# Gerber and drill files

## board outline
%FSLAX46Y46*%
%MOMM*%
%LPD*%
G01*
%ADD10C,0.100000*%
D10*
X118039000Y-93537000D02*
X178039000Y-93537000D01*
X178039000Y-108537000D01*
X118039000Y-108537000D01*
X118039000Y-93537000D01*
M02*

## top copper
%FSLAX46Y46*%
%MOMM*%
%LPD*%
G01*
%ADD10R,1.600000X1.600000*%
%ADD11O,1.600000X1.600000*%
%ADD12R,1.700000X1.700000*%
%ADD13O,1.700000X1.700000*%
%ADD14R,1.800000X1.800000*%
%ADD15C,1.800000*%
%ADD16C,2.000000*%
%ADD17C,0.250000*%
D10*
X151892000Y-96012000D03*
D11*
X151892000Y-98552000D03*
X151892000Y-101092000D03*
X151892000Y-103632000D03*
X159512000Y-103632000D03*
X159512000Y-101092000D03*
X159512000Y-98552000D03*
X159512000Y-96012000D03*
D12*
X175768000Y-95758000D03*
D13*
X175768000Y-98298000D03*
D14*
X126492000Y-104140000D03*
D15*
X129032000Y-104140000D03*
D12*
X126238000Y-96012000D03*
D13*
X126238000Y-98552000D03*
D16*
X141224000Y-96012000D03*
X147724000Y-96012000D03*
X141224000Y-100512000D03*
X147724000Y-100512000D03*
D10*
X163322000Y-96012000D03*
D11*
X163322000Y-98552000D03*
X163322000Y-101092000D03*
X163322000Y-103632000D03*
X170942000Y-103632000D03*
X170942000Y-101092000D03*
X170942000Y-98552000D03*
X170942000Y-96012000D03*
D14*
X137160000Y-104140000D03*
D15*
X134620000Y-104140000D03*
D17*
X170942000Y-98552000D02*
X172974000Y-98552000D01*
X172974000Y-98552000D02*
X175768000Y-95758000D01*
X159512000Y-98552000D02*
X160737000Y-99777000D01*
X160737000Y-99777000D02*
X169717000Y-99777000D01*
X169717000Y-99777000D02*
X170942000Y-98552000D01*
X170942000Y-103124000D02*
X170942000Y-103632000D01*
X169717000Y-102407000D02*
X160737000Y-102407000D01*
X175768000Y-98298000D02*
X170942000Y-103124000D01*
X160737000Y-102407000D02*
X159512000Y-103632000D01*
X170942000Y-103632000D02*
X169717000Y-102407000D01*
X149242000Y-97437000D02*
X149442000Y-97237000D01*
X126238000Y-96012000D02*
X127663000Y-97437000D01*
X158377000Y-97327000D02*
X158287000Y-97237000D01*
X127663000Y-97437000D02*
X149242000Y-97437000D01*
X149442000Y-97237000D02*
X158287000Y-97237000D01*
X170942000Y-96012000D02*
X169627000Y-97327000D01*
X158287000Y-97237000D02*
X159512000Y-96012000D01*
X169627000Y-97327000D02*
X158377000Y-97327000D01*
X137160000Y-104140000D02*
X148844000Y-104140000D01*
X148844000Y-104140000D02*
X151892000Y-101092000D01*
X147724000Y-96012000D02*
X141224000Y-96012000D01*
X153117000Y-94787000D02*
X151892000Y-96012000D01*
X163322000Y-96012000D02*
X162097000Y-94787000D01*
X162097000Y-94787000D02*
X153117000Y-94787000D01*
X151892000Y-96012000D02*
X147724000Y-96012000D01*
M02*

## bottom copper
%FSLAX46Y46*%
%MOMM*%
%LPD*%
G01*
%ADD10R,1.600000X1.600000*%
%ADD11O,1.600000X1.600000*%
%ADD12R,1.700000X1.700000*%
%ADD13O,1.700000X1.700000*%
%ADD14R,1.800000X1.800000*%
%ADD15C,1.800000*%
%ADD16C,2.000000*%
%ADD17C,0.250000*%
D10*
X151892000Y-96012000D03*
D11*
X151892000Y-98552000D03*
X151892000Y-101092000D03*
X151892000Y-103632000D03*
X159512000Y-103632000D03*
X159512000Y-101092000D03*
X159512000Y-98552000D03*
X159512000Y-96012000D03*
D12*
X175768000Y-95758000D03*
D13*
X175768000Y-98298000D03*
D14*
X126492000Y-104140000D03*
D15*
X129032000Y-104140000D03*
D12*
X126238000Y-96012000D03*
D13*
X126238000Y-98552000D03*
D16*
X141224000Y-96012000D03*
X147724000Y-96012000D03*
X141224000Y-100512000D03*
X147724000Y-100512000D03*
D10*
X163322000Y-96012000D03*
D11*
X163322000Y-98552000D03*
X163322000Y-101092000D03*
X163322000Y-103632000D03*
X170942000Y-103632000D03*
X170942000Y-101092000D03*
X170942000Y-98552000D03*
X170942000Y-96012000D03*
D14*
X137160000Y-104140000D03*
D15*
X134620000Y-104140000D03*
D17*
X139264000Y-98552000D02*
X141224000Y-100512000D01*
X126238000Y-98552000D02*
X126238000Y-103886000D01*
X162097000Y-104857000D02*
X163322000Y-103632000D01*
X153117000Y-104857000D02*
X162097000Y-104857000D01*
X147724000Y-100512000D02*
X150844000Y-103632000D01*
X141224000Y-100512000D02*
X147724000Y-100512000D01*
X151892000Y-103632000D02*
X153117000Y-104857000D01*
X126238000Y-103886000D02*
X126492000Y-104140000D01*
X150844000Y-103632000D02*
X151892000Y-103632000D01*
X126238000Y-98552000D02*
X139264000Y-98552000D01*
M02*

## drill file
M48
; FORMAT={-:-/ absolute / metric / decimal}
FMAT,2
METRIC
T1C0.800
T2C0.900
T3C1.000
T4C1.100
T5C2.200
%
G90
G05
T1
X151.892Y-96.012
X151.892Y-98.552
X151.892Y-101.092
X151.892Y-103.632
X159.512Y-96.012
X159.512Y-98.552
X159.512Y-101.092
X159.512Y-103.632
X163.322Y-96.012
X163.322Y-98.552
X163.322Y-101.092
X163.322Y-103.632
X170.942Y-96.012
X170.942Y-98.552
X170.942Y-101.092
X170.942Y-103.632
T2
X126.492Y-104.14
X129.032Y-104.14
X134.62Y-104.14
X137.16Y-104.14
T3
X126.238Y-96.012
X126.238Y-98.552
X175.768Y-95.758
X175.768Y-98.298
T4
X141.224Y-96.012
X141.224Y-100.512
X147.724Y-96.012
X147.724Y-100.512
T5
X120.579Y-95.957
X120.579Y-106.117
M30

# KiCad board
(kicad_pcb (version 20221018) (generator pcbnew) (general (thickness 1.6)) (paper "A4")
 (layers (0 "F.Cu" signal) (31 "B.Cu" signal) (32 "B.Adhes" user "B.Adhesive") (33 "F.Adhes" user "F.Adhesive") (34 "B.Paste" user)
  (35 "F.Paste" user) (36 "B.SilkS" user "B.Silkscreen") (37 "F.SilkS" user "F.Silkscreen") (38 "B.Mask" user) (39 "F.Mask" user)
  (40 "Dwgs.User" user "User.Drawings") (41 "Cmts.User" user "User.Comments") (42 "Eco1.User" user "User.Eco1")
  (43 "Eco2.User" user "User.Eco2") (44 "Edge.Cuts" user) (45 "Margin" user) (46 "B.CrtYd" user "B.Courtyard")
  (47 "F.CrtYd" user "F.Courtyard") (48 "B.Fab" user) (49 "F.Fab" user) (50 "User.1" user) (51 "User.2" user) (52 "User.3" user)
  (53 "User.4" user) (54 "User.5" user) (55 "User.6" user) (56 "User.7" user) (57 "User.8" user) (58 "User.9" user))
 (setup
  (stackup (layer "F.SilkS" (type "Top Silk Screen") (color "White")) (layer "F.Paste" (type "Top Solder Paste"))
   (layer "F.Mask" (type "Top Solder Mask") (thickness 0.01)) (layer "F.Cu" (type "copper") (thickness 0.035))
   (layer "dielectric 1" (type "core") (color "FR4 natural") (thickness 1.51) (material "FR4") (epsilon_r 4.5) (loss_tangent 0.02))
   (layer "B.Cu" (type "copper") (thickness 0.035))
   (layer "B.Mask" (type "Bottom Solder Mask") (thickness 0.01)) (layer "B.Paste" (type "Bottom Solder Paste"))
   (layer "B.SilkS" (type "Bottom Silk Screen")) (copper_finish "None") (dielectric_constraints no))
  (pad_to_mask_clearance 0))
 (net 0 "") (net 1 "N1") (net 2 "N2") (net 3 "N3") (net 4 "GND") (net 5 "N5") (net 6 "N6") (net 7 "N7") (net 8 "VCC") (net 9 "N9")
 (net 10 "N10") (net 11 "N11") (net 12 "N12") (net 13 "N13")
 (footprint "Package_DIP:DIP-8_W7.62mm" (layer "F.Cu") (at 151.892 96.012)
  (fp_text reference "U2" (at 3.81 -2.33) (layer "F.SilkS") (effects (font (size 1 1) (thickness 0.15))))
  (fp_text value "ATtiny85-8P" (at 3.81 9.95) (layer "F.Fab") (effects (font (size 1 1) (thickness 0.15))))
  (pad "1" thru_hole rect (at 0 0) (size 1.6 1.6) (drill 0.8) (layers "*.Cu" "*.Mask") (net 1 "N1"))
  (pad "2" thru_hole oval (at 0 2.54) (size 1.6 1.6) (drill 0.8) (layers "*.Cu" "*.Mask") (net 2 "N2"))
  (pad "3" thru_hole oval (at 0 5.08) (size 1.6 1.6) (drill 0.8) (layers "*.Cu" "*.Mask") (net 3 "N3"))
  (pad "4" thru_hole oval (at 0 7.62) (size 1.6 1.6) (drill 0.8) (layers "*.Cu" "*.Mask") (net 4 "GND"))
  (pad "5" thru_hole oval (at 7.62 7.62) (size 1.6 1.6) (drill 0.8) (layers "*.Cu" "*.Mask") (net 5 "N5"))
  (pad "6" thru_hole oval (at 7.62 5.08) (size 1.6 1.6) (drill 0.8) (layers "*.Cu" "*.Mask") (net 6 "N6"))
  (pad "7" thru_hole oval (at 7.62 2.54) (size 1.6 1.6) (drill 0.8) (layers "*.Cu" "*.Mask") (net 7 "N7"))
  (pad "8" thru_hole oval (at 7.62 0) (size 1.6 1.6) (drill 0.8) (layers "*.Cu" "*.Mask") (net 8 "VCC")))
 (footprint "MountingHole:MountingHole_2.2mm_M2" (layer "F.Cu") (at 120.579 95.957 -90)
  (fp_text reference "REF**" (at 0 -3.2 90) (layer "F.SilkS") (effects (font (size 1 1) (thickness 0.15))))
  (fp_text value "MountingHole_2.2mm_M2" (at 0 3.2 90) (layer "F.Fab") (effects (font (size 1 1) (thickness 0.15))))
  (pad "" np_thru_hole circle (at 0 0 270) (size 2.2 2.2) (drill 2.2) (layers "*.Cu" "*.Mask")))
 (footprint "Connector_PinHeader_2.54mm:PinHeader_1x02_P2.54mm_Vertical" (layer "F.Cu") (at 175.768 95.758)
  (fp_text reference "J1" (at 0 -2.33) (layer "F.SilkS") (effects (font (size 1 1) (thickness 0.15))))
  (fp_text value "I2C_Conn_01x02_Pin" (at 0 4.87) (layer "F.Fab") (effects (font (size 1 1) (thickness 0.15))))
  (pad "1" thru_hole rect (at 0 0) (size 1.7 1.7) (drill 1) (layers "*.Cu" "*.Mask") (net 7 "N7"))
  (pad "2" thru_hole oval (at 0 2.54) (size 1.7 1.7) (drill 1) (layers "*.Cu" "*.Mask") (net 5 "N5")))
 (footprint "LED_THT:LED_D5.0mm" (layer "F.Cu") (at 126.492 104.14)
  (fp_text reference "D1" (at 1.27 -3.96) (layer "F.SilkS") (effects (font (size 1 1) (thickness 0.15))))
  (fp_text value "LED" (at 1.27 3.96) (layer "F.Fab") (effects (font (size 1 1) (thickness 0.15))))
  (pad "1" thru_hole rect (at 0 0) (size 1.8 1.8) (drill 0.9) (layers "*.Cu" "*.Mask") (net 4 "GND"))
  (pad "2" thru_hole circle (at 2.54 0) (size 1.8 1.8) (drill 0.9) (layers "*.Cu" "*.Mask") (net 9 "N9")))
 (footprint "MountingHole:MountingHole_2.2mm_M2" (layer "F.Cu") (at 120.579 106.117 -90)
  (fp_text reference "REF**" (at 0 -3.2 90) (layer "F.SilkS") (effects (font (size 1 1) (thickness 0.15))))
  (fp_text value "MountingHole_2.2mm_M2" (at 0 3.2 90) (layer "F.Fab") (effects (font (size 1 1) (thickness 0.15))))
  (pad "" np_thru_hole circle (at 0 0 270) (size 2.2 2.2) (drill 2.2) (layers "F&B.Cu" "*.Mask")))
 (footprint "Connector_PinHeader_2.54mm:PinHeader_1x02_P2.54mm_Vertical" (layer "F.Cu") (at 126.238 96.012)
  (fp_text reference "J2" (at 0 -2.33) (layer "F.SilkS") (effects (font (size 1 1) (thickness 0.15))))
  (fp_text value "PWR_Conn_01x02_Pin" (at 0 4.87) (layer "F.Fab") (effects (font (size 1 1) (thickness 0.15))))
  (pad "1" thru_hole rect (at 0 0) (size 1.7 1.7) (drill 1) (layers "*.Cu" "*.Mask") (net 8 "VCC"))
  (pad "2" thru_hole oval (at 0 2.54) (size 1.7 1.7) (drill 1) (layers "*.Cu" "*.Mask") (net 4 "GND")))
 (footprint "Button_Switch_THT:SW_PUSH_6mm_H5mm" (layer "F.Cu") (at 141.224 96.012)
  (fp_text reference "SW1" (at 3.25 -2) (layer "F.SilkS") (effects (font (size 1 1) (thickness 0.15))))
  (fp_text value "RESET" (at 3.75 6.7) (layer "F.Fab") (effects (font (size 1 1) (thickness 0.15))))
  (pad "1" thru_hole circle (at 0 0 90) (size 2 2) (drill 1.1) (layers "*.Cu" "*.Mask") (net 1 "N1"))
  (pad "1" thru_hole circle (at 6.5 0 90) (size 2 2) (drill 1.1) (layers "*.Cu" "*.Mask") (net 1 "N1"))
  (pad "2" thru_hole circle (at 0 4.5 90) (size 2 2) (drill 1.1) (layers "*.Cu" "*.Mask") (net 4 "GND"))
  (pad "2" thru_hole circle (at 6.5 4.5 90) (size 2 2) (drill 1.1) (layers "*.Cu" "*.Mask") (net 4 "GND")))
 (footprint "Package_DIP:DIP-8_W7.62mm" (layer "F.Cu") (at 163.322 96.012)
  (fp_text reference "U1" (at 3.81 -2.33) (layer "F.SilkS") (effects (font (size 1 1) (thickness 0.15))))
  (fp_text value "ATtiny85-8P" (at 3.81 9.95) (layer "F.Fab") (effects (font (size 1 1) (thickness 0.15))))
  (pad "1" thru_hole rect (at 0 0) (size 1.6 1.6) (drill 0.8) (layers "*.Cu" "*.Mask") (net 1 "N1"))
  (pad "2" thru_hole oval (at 0 2.54) (size 1.6 1.6) (drill 0.8) (layers "*.Cu" "*.Mask") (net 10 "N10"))
  (pad "3" thru_hole oval (at 0 5.08) (size 1.6 1.6) (drill 0.8) (layers "*.Cu" "*.Mask") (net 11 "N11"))
  (pad "4" thru_hole oval (at 0 7.62) (size 1.6 1.6) (drill 0.8) (layers "*.Cu" "*.Mask") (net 4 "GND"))
  (pad "5" thru_hole oval (at 7.62 7.62) (size 1.6 1.6) (drill 0.8) (layers "*.Cu" "*.Mask") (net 5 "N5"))
  (pad "6" thru_hole oval (at 7.62 5.08) (size 1.6 1.6) (drill 0.8) (layers "*.Cu" "*.Mask") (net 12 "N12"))
  (pad "7" thru_hole oval (at 7.62 2.54) (size 1.6 1.6) (drill 0.8) (layers "*.Cu" "*.Mask") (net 7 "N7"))
  (pad "8" thru_hole oval (at 7.62 0) (size 1.6 1.6) (drill 0.8) (layers "*.Cu" "*.Mask") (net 8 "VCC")))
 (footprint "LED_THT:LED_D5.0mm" (layer "F.Cu") (at 137.16 104.14 180)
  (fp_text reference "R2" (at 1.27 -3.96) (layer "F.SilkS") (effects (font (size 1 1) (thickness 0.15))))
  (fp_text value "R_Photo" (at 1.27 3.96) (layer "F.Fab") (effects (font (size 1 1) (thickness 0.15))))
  (pad "1" thru_hole rect (at 0 0 180) (size 1.8 1.8) (drill 0.9) (layers "*.Cu" "*.Mask") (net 3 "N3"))
  (pad "2" thru_hole circle (at 2.54 0 180) (size 1.8 1.8) (drill 0.9) (layers "*.Cu" "*.Mask") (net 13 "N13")))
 (gr_rect locked (start 118.039 93.537) (end 178.039 108.537) (stroke (width 0.1) (type default)) (fill none) (layer "Edge.Cuts"))
 (segment (start 170.942 98.552) (end 172.974 98.552) (width 0.25) (layer "F.Cu") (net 7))
 (segment (start 172.974 98.552) (end 175.768 95.758) (width 0.25) (layer "F.Cu") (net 7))
 (segment (start 159.512 98.552) (end 160.737 99.777) (width 0.25) (layer "F.Cu") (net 7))
 (segment (start 160.737 99.777) (end 169.717 99.777) (width 0.25) (layer "F.Cu") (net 7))
 (segment (start 169.717 99.777) (end 170.942 98.552) (width 0.25) (layer "F.Cu") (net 7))
 (segment (start 170.942 103.124) (end 170.942 103.632) (width 0.25) (layer "F.Cu") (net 5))
 (segment (start 169.717 102.407) (end 160.737 102.407) (width 0.25) (layer "F.Cu") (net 5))
 (segment (start 175.768 98.298) (end 170.942 103.124) (width 0.25) (layer "F.Cu") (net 5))
 (segment (start 160.737 102.407) (end 159.512 103.632) (width 0.25) (layer "F.Cu") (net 5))
 (segment (start 170.942 103.632) (end 169.717 102.407) (width 0.25) (layer "F.Cu") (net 5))
 (segment (start 139.264 98.552) (end 141.224 100.512) (width 0.25) (layer "B.Cu") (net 4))
 (segment (start 126.238 98.552) (end 126.238 103.886) (width 0.25) (layer "B.Cu") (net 4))
 (segment (start 162.097 104.857) (end 163.322 103.632) (width 0.25) (layer "B.Cu") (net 4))
 (segment (start 153.117 104.857) (end 162.097 104.857) (width 0.25) (layer "B.Cu") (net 4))
 (segment (start 147.724 100.512) (end 150.844 103.632) (width 0.25) (layer "B.Cu") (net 4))
 (segment (start 141.224 100.512) (end 147.724 100.512) (width 0.25) (layer "B.Cu") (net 4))
 (segment (start 151.892 103.632) (end 153.117 104.857) (width 0.25) (layer "B.Cu") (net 4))
 (segment (start 126.238 103.886) (end 126.492 104.14) (width 0.25) (layer "B.Cu") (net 4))
 (segment (start 150.844 103.632) (end 151.892 103.632) (width 0.25) (layer "B.Cu") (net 4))
 (segment (start 126.238 98.552) (end 139.264 98.552) (width 0.25) (layer "B.Cu") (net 4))
 (segment (start 149.242 97.437) (end 149.442 97.237) (width 0.25) (layer "F.Cu") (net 8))
 (segment (start 126.238 96.012) (end 127.663 97.437) (width 0.25) (layer "F.Cu") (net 8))
 (segment (start 158.377 97.327) (end 158.287 97.237) (width 0.25) (layer "F.Cu") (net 8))
 (segment (start 127.663 97.437) (end 149.242 97.437) (width 0.25) (layer "F.Cu") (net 8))
 (segment (start 149.442 97.237) (end 158.287 97.237) (width 0.25) (layer "F.Cu") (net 8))
 (segment (start 170.942 96.012) (end 169.627 97.327) (width 0.25) (layer "F.Cu") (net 8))
 (segment (start 158.287 97.237) (end 159.512 96.012) (width 0.25) (layer "F.Cu") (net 8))
 (segment (start 169.627 97.327) (end 158.377 97.327) (width 0.25) (layer "F.Cu") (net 8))
 (segment (start 137.16 104.14) (end 148.844 104.14) (width 0.25) (layer "F.Cu") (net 3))
 (segment (start 148.844 104.14) (end 151.892 101.092) (width 0.25) (layer "F.Cu") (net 3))
 (segment (start 147.724 96.012) (end 141.224 96.012) (width 0.25) (layer "F.Cu") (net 1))
 (segment (start 153.117 94.787) (end 151.892 96.012) (width 0.25) (layer "F.Cu") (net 1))
 (segment (start 163.322 96.012) (end 162.097 94.787) (width 0.25) (layer "F.Cu") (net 1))
 (segment (start 162.097 94.787) (end 153.117 94.787) (width 0.25) (layer "F.Cu") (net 1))
 (segment (start 151.892 96.012) (end 147.724 96.012) (width 0.25) (layer "F.Cu") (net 1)))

